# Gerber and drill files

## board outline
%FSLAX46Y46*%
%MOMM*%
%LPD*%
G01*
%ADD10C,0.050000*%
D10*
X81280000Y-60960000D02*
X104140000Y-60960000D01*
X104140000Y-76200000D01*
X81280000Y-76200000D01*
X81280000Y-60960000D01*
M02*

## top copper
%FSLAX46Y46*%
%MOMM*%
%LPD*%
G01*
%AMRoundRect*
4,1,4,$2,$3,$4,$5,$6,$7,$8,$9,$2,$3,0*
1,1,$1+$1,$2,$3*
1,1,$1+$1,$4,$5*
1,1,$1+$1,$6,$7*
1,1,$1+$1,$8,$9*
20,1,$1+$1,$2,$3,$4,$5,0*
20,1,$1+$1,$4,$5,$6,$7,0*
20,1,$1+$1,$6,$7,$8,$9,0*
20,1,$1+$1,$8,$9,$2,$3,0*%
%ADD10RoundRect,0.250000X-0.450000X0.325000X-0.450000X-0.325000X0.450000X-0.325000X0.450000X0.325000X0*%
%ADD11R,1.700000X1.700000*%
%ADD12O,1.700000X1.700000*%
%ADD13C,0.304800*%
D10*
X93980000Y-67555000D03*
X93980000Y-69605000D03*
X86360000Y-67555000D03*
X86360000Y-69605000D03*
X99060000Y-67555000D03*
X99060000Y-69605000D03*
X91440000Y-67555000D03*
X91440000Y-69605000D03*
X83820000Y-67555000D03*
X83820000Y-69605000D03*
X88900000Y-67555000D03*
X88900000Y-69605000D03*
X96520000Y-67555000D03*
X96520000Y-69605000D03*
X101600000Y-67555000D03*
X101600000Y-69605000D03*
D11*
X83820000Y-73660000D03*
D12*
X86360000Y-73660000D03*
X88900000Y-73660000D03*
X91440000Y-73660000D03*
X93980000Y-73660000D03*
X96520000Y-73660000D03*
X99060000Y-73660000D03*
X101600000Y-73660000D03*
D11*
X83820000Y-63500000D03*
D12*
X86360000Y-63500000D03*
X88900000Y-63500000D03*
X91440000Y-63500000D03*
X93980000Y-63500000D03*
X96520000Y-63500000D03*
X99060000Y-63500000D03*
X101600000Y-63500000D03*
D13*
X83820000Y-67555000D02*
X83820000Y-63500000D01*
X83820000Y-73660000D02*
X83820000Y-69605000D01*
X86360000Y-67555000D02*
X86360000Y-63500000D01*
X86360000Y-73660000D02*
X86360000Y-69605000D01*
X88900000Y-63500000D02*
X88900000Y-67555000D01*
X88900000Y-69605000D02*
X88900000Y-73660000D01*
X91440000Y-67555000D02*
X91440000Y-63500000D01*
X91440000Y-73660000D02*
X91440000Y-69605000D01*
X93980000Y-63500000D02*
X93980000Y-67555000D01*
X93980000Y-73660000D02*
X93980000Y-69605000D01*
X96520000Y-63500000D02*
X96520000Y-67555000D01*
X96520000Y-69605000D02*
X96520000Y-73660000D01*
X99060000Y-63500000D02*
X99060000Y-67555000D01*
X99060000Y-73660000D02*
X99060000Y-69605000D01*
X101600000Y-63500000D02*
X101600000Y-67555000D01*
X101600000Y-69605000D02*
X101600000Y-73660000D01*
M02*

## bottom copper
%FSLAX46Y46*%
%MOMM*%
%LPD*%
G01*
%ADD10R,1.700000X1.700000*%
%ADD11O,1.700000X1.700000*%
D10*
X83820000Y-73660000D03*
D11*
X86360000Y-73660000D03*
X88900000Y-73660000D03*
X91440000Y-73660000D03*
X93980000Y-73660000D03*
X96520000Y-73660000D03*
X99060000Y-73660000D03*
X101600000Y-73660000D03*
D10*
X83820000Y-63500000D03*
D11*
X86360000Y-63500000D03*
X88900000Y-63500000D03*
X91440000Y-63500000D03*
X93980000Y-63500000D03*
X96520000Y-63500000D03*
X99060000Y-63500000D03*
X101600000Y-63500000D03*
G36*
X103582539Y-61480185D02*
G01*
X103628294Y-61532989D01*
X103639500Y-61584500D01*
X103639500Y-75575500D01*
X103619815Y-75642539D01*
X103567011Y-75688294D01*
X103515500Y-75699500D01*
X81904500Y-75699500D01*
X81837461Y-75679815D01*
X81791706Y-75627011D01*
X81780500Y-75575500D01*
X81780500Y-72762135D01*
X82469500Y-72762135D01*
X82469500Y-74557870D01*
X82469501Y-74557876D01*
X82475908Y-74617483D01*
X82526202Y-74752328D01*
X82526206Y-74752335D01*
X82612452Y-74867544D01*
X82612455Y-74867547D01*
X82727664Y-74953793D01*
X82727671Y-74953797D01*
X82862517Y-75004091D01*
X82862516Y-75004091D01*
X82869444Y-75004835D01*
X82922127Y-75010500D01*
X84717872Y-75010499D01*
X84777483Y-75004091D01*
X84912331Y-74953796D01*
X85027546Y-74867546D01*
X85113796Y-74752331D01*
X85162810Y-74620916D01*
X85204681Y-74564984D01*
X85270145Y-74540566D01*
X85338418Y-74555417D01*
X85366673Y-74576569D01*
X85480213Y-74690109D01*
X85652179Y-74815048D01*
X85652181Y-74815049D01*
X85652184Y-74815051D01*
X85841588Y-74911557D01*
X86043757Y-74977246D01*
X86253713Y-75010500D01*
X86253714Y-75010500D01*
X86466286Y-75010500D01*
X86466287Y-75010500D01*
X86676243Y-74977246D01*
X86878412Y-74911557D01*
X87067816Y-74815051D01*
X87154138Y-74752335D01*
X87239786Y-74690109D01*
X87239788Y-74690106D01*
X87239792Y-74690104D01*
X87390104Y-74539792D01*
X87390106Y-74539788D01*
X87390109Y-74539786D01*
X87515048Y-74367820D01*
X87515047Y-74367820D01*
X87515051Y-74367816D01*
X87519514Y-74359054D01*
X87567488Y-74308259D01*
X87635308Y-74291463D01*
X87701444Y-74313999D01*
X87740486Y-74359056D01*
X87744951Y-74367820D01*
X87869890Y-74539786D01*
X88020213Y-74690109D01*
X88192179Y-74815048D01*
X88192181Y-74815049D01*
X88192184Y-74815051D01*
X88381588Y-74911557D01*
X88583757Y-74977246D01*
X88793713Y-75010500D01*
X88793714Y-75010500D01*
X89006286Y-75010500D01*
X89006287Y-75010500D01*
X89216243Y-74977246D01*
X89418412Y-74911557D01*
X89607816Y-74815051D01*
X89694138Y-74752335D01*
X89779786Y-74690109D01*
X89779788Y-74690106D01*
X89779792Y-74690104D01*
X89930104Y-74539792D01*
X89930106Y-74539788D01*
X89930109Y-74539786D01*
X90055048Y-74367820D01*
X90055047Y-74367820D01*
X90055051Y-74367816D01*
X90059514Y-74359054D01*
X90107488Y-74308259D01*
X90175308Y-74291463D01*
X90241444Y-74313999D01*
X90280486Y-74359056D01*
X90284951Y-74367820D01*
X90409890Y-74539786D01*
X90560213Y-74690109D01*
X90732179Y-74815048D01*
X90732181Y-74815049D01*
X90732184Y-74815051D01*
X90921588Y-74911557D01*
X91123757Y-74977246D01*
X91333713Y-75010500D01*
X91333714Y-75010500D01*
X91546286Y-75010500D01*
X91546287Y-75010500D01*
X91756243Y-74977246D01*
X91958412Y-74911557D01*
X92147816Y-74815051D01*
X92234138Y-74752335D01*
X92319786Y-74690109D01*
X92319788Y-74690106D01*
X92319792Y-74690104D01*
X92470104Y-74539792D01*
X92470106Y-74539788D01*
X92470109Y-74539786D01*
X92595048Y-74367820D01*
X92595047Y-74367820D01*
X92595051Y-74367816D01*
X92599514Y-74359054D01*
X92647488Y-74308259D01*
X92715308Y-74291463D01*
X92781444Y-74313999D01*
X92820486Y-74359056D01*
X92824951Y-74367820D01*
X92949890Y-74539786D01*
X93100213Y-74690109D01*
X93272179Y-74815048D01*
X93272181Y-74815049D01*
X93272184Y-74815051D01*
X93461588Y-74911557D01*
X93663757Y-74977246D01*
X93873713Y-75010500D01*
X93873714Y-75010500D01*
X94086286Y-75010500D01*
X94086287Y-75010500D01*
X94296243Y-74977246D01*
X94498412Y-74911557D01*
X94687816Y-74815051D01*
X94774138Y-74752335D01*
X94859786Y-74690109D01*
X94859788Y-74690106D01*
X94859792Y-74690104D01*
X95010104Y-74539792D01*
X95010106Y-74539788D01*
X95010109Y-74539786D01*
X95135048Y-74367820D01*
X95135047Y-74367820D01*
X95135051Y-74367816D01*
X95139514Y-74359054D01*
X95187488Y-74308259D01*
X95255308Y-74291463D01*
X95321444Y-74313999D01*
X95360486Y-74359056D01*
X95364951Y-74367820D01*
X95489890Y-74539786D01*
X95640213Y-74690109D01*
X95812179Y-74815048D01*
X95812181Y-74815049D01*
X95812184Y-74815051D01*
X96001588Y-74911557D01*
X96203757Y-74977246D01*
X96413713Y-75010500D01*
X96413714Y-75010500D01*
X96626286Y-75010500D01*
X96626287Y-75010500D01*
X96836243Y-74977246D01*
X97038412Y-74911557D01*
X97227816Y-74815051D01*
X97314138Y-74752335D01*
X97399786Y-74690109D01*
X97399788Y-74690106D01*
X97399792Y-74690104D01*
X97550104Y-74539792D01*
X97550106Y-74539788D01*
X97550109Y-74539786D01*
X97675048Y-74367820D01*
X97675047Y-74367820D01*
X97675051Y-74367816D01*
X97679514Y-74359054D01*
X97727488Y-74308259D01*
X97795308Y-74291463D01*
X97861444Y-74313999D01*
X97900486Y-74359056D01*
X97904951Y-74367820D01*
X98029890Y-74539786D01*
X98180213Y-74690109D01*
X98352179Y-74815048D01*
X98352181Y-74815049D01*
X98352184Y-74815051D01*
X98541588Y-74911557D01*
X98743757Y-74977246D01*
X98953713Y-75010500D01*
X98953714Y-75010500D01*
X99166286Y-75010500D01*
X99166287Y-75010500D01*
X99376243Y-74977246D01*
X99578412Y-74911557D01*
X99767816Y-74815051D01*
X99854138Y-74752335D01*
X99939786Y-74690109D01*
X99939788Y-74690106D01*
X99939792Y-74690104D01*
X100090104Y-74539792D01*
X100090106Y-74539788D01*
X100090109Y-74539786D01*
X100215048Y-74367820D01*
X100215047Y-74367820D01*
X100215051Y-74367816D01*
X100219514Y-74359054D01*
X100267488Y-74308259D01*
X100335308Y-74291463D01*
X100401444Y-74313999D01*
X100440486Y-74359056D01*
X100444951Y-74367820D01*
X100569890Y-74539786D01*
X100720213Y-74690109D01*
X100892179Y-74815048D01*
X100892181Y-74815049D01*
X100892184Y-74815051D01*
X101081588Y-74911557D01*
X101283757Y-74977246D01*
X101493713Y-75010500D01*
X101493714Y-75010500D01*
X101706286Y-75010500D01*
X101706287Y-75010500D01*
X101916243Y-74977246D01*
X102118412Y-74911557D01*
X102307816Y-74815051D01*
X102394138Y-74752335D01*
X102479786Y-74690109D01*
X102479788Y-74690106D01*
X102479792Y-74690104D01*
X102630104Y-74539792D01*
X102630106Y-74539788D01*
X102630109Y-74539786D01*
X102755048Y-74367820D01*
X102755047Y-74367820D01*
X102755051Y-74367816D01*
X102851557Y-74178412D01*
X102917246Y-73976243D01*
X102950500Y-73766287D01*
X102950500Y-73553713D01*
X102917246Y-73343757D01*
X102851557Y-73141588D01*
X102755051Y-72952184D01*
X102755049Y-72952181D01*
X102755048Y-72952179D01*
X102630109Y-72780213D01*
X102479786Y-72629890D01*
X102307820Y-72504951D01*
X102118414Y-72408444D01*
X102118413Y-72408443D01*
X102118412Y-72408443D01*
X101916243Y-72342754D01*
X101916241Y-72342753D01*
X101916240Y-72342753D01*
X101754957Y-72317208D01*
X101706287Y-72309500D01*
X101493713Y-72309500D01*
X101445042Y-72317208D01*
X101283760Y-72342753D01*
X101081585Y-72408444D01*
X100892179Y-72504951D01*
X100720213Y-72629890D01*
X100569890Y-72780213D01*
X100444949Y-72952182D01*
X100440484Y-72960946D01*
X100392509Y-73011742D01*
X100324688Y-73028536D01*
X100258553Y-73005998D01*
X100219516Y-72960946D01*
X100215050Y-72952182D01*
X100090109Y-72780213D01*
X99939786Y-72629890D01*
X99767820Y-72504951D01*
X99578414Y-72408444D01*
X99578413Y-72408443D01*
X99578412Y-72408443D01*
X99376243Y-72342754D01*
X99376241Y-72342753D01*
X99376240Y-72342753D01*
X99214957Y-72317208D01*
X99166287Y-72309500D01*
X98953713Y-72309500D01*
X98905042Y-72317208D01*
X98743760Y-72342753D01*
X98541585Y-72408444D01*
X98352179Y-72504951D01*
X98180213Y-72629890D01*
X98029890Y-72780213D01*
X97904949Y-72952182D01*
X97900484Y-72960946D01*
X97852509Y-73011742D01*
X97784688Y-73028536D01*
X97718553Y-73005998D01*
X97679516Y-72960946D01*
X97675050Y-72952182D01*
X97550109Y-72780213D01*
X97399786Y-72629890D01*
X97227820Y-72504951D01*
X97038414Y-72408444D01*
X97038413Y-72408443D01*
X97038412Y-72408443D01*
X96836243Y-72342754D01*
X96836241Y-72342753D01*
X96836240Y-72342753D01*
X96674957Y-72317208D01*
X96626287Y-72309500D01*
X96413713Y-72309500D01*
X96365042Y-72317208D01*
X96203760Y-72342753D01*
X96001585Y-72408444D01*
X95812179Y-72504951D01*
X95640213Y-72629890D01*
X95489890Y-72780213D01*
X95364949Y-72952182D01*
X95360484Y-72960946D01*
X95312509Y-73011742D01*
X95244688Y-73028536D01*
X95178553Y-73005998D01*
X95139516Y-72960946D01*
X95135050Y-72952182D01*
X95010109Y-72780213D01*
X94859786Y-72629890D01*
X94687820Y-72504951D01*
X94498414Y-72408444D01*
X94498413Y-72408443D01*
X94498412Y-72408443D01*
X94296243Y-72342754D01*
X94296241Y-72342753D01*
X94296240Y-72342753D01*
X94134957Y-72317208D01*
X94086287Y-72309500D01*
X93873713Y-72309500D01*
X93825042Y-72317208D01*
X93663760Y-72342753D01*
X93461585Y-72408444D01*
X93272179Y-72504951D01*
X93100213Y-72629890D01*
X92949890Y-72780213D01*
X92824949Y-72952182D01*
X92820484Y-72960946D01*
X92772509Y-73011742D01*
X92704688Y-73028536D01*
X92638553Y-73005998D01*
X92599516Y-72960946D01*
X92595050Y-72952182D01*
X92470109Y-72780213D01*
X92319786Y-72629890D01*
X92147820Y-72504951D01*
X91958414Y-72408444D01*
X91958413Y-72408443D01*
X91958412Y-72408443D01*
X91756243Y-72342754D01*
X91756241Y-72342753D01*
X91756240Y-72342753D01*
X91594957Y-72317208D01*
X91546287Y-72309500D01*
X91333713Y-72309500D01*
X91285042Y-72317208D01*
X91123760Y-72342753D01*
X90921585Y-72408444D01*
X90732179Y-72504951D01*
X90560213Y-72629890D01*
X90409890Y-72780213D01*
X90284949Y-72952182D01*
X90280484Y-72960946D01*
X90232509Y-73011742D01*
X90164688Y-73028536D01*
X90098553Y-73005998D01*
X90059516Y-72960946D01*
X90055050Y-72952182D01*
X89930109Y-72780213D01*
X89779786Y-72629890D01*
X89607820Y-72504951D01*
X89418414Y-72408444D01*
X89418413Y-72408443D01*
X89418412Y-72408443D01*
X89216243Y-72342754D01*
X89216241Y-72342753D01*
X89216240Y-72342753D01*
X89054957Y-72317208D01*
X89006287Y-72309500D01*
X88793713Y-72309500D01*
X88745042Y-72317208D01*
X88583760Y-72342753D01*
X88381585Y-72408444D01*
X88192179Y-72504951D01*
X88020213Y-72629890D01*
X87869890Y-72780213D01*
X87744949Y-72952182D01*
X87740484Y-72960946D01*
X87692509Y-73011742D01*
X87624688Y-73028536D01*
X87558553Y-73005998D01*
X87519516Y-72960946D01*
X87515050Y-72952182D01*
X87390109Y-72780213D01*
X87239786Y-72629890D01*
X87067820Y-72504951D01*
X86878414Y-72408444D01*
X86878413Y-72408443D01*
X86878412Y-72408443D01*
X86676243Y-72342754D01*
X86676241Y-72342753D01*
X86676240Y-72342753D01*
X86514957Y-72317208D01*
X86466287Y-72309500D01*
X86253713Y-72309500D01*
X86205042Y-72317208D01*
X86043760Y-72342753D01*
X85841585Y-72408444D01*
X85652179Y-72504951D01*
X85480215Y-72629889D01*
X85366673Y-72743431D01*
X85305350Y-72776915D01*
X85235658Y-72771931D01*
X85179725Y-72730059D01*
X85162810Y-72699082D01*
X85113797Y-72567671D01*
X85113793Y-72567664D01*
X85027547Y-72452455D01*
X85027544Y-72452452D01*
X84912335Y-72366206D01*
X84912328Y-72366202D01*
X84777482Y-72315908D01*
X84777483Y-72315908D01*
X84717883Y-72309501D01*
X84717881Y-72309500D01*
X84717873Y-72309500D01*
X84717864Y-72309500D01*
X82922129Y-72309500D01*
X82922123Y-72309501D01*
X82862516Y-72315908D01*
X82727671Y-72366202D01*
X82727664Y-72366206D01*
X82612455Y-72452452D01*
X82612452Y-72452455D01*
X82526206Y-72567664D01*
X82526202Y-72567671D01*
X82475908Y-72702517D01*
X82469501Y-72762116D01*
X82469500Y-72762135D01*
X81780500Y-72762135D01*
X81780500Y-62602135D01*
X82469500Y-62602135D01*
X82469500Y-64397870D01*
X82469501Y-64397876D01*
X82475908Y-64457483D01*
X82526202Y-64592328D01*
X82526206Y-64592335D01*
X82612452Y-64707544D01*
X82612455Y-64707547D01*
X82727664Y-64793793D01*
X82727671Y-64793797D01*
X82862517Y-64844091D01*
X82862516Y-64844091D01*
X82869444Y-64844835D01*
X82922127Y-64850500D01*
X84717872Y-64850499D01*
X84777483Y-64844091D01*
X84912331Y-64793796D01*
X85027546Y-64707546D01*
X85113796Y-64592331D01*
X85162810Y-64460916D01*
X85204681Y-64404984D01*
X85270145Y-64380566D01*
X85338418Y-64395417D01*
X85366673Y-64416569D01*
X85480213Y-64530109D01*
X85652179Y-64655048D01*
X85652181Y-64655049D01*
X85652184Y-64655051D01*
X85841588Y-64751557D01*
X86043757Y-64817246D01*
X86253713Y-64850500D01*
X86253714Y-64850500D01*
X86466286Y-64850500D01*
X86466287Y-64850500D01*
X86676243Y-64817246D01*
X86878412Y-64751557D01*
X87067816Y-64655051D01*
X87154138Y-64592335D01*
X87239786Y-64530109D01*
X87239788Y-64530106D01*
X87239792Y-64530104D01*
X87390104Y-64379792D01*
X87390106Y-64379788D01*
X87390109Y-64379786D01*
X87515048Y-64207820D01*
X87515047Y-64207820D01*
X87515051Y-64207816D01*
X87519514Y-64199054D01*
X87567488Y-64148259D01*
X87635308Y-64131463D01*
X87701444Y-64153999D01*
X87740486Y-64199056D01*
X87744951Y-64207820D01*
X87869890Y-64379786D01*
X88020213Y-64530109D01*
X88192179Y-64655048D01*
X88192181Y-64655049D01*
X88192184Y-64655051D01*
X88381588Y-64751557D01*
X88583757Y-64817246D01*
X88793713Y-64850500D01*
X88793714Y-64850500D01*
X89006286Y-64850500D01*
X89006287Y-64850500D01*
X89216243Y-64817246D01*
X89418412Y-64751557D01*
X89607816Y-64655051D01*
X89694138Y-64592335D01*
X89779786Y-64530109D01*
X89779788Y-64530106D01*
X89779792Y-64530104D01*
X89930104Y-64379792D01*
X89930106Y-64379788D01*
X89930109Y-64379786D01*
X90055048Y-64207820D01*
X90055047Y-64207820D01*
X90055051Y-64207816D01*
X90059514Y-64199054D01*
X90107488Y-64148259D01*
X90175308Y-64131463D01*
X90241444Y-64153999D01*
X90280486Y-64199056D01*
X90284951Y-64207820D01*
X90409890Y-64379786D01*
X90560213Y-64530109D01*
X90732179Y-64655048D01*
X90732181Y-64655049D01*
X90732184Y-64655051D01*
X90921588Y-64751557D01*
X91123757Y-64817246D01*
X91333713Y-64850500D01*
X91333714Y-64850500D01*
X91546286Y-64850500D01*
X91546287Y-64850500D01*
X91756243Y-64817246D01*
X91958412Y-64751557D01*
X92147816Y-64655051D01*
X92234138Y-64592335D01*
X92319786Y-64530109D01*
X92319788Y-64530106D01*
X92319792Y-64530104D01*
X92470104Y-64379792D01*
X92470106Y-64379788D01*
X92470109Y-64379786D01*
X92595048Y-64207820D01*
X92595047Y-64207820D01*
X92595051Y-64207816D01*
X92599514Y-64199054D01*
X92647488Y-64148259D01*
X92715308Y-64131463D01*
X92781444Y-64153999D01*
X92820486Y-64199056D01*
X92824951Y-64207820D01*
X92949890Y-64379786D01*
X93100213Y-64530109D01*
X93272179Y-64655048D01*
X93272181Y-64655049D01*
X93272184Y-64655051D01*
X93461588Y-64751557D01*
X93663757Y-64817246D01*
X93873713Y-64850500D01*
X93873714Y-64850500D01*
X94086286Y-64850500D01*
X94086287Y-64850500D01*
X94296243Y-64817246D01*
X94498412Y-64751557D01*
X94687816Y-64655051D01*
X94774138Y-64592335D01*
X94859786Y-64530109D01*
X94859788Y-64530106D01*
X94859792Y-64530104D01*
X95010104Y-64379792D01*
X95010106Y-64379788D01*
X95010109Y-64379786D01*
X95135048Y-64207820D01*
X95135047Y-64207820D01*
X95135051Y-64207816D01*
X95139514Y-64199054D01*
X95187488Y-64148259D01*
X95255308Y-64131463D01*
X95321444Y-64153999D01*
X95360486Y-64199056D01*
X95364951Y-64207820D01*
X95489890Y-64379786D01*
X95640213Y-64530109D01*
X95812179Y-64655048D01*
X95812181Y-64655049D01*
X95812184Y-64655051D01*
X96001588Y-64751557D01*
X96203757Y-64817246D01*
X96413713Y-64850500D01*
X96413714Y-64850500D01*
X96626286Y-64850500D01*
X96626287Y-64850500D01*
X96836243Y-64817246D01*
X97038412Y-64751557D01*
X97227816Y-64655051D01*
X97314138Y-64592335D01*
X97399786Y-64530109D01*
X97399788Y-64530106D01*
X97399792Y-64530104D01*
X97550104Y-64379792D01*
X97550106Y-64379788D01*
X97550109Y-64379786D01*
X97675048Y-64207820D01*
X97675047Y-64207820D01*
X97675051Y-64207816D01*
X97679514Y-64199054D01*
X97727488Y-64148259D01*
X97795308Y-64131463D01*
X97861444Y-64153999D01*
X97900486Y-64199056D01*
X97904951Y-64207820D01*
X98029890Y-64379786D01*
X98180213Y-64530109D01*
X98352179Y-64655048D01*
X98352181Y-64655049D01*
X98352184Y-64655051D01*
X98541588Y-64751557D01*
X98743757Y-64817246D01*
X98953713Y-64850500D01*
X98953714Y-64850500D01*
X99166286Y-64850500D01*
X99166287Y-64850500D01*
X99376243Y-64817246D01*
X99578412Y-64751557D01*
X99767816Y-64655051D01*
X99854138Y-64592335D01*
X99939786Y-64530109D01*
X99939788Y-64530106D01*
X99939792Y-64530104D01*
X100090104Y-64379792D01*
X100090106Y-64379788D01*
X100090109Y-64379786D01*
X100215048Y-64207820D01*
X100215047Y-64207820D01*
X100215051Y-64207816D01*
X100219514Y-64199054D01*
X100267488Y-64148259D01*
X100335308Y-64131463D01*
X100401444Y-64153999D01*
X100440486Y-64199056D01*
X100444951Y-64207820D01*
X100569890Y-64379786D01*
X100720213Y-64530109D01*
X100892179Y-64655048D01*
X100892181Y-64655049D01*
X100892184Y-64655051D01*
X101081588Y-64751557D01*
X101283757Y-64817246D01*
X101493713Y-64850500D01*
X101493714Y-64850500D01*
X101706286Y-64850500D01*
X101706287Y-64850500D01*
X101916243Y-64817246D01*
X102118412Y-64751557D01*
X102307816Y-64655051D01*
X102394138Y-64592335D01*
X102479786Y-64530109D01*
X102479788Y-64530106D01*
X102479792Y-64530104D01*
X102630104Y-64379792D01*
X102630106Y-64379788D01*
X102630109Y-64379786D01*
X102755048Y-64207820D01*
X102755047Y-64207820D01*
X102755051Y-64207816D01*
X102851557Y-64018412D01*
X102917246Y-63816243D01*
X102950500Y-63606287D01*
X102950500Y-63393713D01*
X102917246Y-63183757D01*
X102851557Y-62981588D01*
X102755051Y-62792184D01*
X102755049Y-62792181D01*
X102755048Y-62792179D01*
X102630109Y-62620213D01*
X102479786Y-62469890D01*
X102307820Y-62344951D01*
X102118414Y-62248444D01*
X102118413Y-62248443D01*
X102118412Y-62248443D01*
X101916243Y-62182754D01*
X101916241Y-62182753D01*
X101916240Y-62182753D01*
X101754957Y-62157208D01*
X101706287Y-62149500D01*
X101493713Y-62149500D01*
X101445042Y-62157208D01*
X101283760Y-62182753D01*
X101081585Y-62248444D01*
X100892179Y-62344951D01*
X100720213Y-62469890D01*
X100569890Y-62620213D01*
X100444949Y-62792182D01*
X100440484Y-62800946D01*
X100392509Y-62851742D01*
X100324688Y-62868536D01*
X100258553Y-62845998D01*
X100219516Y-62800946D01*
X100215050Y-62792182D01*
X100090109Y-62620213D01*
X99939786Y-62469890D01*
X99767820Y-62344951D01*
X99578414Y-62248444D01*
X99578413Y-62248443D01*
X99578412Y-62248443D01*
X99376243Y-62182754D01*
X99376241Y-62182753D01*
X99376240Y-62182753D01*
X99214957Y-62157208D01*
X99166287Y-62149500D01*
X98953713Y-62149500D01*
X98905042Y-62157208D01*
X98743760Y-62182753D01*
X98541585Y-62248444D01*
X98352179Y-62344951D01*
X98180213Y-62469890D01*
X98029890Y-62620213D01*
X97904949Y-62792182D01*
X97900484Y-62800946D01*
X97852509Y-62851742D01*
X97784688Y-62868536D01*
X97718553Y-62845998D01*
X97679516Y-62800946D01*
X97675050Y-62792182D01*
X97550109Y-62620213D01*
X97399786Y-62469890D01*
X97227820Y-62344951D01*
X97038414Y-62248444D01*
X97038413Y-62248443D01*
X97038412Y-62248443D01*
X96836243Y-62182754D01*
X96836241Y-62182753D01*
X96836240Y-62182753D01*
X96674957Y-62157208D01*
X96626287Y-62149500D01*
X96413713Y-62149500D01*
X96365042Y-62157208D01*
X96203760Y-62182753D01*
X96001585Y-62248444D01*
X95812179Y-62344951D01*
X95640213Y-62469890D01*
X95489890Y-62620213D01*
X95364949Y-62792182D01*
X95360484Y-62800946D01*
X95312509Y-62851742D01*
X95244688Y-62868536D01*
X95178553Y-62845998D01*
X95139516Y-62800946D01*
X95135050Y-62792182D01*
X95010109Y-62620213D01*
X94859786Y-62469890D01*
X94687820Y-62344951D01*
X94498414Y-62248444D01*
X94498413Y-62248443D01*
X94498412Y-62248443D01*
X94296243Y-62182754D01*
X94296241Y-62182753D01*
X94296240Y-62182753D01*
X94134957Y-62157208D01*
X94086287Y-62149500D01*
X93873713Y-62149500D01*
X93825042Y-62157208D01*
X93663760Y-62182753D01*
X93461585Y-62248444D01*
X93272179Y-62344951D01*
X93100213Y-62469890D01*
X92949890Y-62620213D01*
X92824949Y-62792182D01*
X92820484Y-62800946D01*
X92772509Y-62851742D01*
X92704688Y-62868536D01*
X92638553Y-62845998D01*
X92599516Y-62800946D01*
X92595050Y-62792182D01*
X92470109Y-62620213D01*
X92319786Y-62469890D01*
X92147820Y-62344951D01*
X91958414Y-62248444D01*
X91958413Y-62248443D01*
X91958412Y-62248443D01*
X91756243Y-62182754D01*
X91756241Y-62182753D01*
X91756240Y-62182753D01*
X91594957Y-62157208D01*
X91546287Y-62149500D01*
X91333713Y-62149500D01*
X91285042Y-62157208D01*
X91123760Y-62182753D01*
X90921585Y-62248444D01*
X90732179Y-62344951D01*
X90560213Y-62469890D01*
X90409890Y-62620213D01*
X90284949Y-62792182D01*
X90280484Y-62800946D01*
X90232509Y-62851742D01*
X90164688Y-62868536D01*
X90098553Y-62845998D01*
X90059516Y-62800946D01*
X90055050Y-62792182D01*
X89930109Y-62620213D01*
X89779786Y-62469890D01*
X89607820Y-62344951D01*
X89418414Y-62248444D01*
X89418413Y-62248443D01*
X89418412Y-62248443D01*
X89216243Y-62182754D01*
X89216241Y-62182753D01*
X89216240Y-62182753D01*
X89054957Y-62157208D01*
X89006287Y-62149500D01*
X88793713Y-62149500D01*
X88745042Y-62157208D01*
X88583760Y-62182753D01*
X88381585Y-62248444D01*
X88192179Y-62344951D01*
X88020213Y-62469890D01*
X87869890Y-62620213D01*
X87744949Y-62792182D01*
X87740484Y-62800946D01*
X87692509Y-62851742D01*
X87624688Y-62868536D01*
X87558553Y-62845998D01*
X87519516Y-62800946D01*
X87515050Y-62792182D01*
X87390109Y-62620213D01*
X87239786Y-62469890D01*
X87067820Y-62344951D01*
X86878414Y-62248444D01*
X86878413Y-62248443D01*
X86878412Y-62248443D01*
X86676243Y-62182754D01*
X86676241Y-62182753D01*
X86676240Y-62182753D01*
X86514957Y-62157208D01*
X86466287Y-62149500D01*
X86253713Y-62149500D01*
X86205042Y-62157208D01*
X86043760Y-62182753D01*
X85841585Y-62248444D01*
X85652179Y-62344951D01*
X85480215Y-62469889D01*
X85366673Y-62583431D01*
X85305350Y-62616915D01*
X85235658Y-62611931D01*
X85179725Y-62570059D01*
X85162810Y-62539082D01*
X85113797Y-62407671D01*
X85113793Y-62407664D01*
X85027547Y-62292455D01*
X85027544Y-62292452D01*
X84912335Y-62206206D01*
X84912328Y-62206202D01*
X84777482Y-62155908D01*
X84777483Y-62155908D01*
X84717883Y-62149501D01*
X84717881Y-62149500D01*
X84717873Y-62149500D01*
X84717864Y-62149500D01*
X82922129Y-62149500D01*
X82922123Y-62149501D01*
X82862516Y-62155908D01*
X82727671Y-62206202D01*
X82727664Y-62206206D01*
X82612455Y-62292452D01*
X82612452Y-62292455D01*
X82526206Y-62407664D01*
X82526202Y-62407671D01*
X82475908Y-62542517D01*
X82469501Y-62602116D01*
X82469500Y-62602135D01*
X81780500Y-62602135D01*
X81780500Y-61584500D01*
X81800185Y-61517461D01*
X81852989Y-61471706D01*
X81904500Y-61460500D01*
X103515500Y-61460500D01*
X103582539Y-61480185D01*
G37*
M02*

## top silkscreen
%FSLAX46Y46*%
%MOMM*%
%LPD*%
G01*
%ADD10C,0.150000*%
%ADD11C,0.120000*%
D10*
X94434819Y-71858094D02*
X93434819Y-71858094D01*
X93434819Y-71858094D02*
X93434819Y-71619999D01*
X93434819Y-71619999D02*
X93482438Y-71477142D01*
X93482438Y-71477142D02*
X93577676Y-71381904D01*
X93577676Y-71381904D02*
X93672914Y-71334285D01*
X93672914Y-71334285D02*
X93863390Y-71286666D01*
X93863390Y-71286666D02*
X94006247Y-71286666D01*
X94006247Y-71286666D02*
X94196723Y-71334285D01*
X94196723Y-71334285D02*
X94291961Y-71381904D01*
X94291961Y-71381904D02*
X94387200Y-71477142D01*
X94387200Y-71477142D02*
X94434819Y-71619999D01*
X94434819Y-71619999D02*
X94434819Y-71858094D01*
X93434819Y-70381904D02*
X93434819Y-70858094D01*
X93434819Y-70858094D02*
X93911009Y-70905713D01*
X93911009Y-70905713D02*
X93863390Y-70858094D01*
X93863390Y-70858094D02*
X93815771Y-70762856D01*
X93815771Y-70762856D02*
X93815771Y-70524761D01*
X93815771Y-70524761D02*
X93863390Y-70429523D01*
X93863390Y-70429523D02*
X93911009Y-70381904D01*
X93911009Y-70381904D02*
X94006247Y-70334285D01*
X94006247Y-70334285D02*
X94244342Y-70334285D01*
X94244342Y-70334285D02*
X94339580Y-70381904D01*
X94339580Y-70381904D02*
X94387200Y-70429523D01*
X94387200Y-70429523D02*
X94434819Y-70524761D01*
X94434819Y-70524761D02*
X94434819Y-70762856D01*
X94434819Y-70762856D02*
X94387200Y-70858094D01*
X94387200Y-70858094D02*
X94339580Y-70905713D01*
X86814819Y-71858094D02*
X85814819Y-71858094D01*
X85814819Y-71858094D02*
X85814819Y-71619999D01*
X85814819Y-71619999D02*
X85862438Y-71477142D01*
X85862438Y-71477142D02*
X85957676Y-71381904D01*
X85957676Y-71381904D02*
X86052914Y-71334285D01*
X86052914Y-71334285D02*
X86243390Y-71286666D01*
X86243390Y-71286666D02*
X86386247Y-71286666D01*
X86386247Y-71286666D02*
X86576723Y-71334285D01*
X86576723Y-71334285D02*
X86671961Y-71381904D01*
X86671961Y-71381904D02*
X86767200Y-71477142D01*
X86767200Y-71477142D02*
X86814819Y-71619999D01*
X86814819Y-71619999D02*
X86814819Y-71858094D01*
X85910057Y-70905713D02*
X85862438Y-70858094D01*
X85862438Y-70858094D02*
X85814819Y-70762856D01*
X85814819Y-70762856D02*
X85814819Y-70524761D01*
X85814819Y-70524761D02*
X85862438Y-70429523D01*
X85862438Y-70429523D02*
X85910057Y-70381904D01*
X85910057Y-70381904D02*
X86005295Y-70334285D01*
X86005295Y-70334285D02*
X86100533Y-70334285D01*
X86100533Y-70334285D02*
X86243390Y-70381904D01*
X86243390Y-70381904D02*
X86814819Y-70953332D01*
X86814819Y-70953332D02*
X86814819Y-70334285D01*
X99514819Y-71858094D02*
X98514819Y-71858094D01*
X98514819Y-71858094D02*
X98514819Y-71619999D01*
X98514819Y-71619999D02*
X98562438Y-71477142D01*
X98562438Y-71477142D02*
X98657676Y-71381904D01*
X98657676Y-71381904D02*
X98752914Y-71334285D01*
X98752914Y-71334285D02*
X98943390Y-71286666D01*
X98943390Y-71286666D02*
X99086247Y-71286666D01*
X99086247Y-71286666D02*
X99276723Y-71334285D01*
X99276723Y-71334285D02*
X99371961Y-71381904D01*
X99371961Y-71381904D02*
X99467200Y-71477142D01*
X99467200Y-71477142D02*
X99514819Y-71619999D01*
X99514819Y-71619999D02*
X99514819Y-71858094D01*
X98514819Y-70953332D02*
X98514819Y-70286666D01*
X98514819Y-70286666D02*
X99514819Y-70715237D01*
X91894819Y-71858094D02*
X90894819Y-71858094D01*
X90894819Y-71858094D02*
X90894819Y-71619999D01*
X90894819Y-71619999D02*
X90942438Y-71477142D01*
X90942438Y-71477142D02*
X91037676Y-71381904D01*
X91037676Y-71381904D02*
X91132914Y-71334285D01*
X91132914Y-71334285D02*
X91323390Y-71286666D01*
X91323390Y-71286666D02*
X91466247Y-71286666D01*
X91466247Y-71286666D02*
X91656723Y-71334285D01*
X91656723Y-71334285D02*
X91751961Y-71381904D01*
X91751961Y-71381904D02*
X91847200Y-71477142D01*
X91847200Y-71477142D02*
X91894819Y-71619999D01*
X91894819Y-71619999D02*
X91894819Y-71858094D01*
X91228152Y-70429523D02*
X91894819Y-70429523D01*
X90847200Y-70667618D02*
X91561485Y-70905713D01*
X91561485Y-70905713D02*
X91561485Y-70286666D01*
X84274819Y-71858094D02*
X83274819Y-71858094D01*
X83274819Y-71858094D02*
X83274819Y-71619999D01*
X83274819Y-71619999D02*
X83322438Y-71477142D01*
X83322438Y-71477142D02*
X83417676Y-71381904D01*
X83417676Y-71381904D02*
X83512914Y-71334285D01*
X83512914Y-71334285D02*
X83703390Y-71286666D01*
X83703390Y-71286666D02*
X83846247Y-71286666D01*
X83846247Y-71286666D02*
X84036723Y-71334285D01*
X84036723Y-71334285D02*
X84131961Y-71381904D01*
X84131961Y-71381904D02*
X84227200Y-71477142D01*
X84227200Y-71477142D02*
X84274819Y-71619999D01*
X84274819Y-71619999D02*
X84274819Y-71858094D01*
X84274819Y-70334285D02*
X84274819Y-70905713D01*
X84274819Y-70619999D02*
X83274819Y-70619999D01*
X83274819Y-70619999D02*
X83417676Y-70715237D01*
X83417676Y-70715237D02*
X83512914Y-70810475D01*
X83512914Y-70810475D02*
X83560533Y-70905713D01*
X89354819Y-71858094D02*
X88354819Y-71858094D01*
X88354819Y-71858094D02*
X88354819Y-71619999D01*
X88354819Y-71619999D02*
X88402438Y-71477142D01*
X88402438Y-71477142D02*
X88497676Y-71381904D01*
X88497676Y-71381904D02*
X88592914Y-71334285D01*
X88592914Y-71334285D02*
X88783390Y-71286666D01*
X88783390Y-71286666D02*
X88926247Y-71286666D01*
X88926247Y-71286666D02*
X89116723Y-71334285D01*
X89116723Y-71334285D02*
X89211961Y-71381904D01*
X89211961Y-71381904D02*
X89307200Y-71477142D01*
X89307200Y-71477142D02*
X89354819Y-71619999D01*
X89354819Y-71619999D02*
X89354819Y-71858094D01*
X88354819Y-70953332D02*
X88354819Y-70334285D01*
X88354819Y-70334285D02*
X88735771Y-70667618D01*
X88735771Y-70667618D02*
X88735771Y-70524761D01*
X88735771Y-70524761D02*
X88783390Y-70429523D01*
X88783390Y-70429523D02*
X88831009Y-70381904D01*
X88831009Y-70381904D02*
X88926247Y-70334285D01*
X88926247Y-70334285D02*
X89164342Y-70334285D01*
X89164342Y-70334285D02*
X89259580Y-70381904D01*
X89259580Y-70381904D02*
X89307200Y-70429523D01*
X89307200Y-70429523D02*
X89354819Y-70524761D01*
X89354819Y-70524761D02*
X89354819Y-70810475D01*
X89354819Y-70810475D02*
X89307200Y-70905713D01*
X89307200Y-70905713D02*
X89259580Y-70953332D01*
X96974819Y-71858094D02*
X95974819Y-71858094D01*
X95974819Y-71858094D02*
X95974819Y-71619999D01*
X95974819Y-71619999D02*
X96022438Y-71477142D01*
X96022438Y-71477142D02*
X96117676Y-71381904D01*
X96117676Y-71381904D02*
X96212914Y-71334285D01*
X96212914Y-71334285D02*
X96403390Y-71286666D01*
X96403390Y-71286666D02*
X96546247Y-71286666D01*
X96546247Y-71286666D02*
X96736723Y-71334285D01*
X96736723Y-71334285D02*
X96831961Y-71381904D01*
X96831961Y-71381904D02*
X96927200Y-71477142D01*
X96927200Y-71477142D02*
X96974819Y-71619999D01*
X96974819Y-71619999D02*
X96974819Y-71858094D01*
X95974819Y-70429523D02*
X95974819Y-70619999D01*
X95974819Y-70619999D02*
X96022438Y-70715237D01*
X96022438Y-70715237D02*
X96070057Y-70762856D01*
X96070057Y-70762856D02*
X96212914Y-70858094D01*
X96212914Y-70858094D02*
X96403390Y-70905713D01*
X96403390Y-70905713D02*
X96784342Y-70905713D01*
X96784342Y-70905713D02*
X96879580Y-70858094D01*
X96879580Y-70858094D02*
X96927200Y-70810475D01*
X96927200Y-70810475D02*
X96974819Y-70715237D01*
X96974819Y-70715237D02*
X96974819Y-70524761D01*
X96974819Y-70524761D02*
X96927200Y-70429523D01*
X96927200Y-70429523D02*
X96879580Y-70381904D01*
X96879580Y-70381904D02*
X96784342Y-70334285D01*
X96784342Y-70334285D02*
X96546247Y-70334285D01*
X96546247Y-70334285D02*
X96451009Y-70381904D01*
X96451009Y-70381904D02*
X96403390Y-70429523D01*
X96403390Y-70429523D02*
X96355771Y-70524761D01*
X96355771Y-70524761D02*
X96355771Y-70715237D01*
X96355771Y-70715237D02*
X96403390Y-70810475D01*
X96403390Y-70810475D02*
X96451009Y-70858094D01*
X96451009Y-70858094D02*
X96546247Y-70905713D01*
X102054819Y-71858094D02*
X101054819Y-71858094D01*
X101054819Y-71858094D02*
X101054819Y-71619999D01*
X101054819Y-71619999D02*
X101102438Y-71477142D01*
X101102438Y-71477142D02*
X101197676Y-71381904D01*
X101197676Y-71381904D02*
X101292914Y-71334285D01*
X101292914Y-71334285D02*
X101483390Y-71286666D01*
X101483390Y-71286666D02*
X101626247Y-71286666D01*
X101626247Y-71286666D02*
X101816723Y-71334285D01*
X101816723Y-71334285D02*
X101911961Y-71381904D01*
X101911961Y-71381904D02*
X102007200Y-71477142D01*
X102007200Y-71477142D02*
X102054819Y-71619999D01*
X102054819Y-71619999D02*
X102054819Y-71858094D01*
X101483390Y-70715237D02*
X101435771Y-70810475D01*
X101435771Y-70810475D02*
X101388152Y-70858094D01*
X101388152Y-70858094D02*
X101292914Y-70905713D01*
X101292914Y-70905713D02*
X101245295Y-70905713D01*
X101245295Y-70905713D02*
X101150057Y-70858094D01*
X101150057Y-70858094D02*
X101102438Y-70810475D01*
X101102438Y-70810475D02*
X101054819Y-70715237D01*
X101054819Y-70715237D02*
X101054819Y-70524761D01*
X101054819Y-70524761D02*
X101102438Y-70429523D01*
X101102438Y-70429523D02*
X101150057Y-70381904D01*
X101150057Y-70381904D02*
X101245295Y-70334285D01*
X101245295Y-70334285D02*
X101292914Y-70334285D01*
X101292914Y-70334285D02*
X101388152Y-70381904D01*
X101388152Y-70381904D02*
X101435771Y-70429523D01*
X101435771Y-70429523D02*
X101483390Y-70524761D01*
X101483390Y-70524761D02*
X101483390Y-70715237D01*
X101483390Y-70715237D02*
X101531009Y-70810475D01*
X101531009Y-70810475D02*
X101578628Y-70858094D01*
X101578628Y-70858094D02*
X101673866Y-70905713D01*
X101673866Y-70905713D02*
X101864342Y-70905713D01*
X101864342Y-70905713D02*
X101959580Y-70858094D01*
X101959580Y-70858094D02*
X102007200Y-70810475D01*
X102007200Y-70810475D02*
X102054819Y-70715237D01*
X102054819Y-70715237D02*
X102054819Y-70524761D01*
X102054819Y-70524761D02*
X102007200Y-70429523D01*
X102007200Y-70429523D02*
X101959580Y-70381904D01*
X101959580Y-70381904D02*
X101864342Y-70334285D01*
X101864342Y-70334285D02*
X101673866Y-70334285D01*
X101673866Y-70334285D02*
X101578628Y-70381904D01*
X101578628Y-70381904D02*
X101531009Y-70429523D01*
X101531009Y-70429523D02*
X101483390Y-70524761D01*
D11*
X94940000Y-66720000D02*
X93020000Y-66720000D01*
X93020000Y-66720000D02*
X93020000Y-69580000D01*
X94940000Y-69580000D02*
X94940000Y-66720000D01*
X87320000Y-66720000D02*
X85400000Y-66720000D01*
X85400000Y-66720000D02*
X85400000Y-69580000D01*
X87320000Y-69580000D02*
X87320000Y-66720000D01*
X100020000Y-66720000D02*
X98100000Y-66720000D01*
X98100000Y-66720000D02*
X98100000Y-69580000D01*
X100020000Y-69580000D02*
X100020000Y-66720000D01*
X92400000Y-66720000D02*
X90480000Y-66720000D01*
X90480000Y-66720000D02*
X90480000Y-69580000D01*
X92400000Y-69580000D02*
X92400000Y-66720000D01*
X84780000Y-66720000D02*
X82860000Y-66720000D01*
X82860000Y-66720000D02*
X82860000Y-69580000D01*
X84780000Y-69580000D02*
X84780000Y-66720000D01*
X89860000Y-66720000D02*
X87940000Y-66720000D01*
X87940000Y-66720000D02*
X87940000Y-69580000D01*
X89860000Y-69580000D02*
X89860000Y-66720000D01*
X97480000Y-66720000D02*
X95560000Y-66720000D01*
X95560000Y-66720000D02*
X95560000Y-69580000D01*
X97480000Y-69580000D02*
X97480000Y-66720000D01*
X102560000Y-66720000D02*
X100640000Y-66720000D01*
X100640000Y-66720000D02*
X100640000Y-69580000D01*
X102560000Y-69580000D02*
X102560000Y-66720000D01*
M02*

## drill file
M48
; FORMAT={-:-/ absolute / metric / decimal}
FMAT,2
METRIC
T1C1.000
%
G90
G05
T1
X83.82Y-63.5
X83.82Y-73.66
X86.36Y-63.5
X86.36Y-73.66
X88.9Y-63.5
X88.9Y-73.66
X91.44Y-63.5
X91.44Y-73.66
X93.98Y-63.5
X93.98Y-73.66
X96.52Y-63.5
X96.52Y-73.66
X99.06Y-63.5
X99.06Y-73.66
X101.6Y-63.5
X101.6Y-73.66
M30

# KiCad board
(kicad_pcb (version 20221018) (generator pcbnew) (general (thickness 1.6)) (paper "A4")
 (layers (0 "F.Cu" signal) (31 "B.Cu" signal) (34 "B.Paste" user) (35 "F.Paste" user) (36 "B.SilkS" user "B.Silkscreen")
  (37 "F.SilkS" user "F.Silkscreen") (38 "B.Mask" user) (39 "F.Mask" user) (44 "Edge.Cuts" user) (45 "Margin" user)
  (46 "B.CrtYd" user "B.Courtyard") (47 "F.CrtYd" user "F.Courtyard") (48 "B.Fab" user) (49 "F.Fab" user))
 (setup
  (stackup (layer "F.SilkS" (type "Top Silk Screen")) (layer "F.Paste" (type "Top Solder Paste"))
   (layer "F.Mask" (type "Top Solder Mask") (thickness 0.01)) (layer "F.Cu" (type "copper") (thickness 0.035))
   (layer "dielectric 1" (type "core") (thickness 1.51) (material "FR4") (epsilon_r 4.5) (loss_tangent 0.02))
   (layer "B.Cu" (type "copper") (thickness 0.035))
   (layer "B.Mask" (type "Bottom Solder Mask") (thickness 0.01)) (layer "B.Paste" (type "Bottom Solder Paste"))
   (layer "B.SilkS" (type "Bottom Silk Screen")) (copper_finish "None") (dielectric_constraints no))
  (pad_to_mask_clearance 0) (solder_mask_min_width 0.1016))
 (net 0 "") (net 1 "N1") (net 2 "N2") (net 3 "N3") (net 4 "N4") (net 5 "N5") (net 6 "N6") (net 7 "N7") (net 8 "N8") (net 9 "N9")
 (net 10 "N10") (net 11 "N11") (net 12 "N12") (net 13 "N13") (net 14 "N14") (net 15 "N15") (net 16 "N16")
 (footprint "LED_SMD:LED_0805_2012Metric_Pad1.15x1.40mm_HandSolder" (layer "F.Cu") (at 93.98 68.58 -90)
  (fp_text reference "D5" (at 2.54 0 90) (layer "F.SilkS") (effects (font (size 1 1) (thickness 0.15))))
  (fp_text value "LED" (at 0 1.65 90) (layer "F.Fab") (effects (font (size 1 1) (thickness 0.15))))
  (fp_line (start -1.86 -0.96) (end -1.86 0.96) (stroke (width 0.12) (type solid)) (layer "F.SilkS"))
  (fp_line (start -1.86 0.96) (end 1 0.96) (stroke (width 0.12) (type solid)) (layer "F.SilkS"))
  (fp_line (start 1 -0.96) (end -1.86 -0.96) (stroke (width 0.12) (type solid)) (layer "F.SilkS"))
  (pad "1" smd roundrect (at -1.025 0 270) (size 1.15 1.4) (layers "F.Cu" "F.Paste" "F.Mask") (roundrect_rratio 0.217391) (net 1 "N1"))
  (pad "2" smd roundrect (at 1.025 0 270) (size 1.15 1.4) (layers "F.Cu" "F.Paste" "F.Mask") (roundrect_rratio 0.217391) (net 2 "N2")))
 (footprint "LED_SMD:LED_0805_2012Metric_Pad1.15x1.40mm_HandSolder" (layer "F.Cu") (at 86.36 68.58 -90)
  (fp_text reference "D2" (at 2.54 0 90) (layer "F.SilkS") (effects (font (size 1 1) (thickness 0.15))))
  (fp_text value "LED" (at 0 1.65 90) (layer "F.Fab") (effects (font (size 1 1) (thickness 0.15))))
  (fp_line (start -1.86 -0.96) (end -1.86 0.96) (stroke (width 0.12) (type solid)) (layer "F.SilkS"))
  (fp_line (start -1.86 0.96) (end 1 0.96) (stroke (width 0.12) (type solid)) (layer "F.SilkS"))
  (fp_line (start 1 -0.96) (end -1.86 -0.96) (stroke (width 0.12) (type solid)) (layer "F.SilkS"))
  (pad "1" smd roundrect (at -1.025 0 270) (size 1.15 1.4) (layers "F.Cu" "F.Paste" "F.Mask") (roundrect_rratio 0.217391) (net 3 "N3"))
  (pad "2" smd roundrect (at 1.025 0 270) (size 1.15 1.4) (layers "F.Cu" "F.Paste" "F.Mask") (roundrect_rratio 0.217391) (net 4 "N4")))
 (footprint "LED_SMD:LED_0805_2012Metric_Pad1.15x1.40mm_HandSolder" (layer "F.Cu") (at 99.06 68.58 -90)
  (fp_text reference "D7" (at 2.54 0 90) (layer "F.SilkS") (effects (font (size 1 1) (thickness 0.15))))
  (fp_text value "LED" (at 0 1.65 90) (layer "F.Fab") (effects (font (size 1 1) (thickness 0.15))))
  (fp_line (start -1.86 -0.96) (end -1.86 0.96) (stroke (width 0.12) (type solid)) (layer "F.SilkS"))
  (fp_line (start -1.86 0.96) (end 1 0.96) (stroke (width 0.12) (type solid)) (layer "F.SilkS"))
  (fp_line (start 1 -0.96) (end -1.86 -0.96) (stroke (width 0.12) (type solid)) (layer "F.SilkS"))
  (pad "1" smd roundrect (at -1.025 0 270) (size 1.15 1.4) (layers "F.Cu" "F.Paste" "F.Mask") (roundrect_rratio 0.217391) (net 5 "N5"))
  (pad "2" smd roundrect (at 1.025 0 270) (size 1.15 1.4) (layers "F.Cu" "F.Paste" "F.Mask") (roundrect_rratio 0.217391) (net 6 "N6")))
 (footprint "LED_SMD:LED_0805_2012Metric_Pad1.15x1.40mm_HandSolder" (layer "F.Cu") (at 91.44 68.58 -90)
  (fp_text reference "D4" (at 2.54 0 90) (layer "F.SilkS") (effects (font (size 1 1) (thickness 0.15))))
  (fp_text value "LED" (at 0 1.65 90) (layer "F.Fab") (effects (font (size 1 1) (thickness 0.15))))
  (fp_line (start -1.86 -0.96) (end -1.86 0.96) (stroke (width 0.12) (type solid)) (layer "F.SilkS"))
  (fp_line (start -1.86 0.96) (end 1 0.96) (stroke (width 0.12) (type solid)) (layer "F.SilkS"))
  (fp_line (start 1 -0.96) (end -1.86 -0.96) (stroke (width 0.12) (type solid)) (layer "F.SilkS"))
  (pad "1" smd roundrect (at -1.025 0 270) (size 1.15 1.4) (layers "F.Cu" "F.Paste" "F.Mask") (roundrect_rratio 0.217391) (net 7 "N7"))
  (pad "2" smd roundrect (at 1.025 0 270) (size 1.15 1.4) (layers "F.Cu" "F.Paste" "F.Mask") (roundrect_rratio 0.217391) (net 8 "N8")))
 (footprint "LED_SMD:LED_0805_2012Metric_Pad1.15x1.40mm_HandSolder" (layer "F.Cu") (at 83.82 68.58 -90)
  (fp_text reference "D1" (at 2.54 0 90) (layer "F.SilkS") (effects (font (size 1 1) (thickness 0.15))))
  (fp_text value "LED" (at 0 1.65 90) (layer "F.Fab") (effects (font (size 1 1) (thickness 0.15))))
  (fp_line (start -1.86 -0.96) (end -1.86 0.96) (stroke (width 0.12) (type solid)) (layer "F.SilkS"))
  (fp_line (start -1.86 0.96) (end 1 0.96) (stroke (width 0.12) (type solid)) (layer "F.SilkS"))
  (fp_line (start 1 -0.96) (end -1.86 -0.96) (stroke (width 0.12) (type solid)) (layer "F.SilkS"))
  (pad "1" smd roundrect (at -1.025 0 270) (size 1.15 1.4) (layers "F.Cu" "F.Paste" "F.Mask") (roundrect_rratio 0.217391) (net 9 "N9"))
  (pad "2" smd roundrect (at 1.025 0 270) (size 1.15 1.4) (layers "F.Cu" "F.Paste" "F.Mask") (roundrect_rratio 0.217391) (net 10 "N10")))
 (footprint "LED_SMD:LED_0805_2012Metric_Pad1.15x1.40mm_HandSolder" (layer "F.Cu") (at 88.9 68.58 -90)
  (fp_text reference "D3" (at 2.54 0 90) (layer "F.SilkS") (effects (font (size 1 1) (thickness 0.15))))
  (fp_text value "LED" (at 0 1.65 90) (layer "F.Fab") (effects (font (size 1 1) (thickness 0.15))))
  (fp_line (start -1.86 -0.96) (end -1.86 0.96) (stroke (width 0.12) (type solid)) (layer "F.SilkS"))
  (fp_line (start -1.86 0.96) (end 1 0.96) (stroke (width 0.12) (type solid)) (layer "F.SilkS"))
  (fp_line (start 1 -0.96) (end -1.86 -0.96) (stroke (width 0.12) (type solid)) (layer "F.SilkS"))
  (pad "1" smd roundrect (at -1.025 0 270) (size 1.15 1.4) (layers "F.Cu" "F.Paste" "F.Mask") (roundrect_rratio 0.217391) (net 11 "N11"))
  (pad "2" smd roundrect (at 1.025 0 270) (size 1.15 1.4) (layers "F.Cu" "F.Paste" "F.Mask") (roundrect_rratio 0.217391) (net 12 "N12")))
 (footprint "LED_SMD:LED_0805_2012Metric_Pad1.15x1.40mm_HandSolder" (layer "F.Cu") (at 96.52 68.58 -90)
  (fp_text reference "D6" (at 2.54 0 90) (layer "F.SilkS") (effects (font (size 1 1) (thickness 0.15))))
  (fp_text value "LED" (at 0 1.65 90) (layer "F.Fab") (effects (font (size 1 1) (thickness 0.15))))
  (fp_line (start -1.86 -0.96) (end -1.86 0.96) (stroke (width 0.12) (type solid)) (layer "F.SilkS"))
  (fp_line (start -1.86 0.96) (end 1 0.96) (stroke (width 0.12) (type solid)) (layer "F.SilkS"))
  (fp_line (start 1 -0.96) (end -1.86 -0.96) (stroke (width 0.12) (type solid)) (layer "F.SilkS"))
  (pad "1" smd roundrect (at -1.025 0 270) (size 1.15 1.4) (layers "F.Cu" "F.Paste" "F.Mask") (roundrect_rratio 0.217391) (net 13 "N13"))
  (pad "2" smd roundrect (at 1.025 0 270) (size 1.15 1.4) (layers "F.Cu" "F.Paste" "F.Mask") (roundrect_rratio 0.217391) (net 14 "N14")))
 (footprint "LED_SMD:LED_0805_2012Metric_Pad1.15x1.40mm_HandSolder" (layer "F.Cu") (at 101.6 68.58 -90)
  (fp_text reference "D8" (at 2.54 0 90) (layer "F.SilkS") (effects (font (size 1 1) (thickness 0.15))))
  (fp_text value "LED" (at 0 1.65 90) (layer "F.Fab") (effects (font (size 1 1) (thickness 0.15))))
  (fp_line (start -1.86 -0.96) (end -1.86 0.96) (stroke (width 0.12) (type solid)) (layer "F.SilkS"))
  (fp_line (start -1.86 0.96) (end 1 0.96) (stroke (width 0.12) (type solid)) (layer "F.SilkS"))
  (fp_line (start 1 -0.96) (end -1.86 -0.96) (stroke (width 0.12) (type solid)) (layer "F.SilkS"))
  (pad "1" smd roundrect (at -1.025 0 270) (size 1.15 1.4) (layers "F.Cu" "F.Paste" "F.Mask") (roundrect_rratio 0.217391) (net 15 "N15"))
  (pad "2" smd roundrect (at 1.025 0 270) (size 1.15 1.4) (layers "F.Cu" "F.Paste" "F.Mask") (roundrect_rratio 0.217391) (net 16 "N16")))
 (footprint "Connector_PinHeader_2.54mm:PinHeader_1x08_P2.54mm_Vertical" (layer "B.Cu") (at 83.82 73.66 -90)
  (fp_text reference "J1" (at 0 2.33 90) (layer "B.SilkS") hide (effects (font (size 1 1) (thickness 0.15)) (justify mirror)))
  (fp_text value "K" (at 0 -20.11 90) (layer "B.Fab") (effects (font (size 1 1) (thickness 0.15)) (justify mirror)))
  (pad "1" thru_hole rect (at 0 0 270) (size 1.7 1.7) (drill 1) (layers "*.Cu" "*.Mask") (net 10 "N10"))
  (pad "2" thru_hole oval (at 0 -2.54 270) (size 1.7 1.7) (drill 1) (layers "*.Cu" "*.Mask") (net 4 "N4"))
  (pad "3" thru_hole oval (at 0 -5.08 270) (size 1.7 1.7) (drill 1) (layers "*.Cu" "*.Mask") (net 12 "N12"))
  (pad "4" thru_hole oval (at 0 -7.62 270) (size 1.7 1.7) (drill 1) (layers "*.Cu" "*.Mask") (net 8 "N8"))
  (pad "5" thru_hole oval (at 0 -10.16 270) (size 1.7 1.7) (drill 1) (layers "*.Cu" "*.Mask") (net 2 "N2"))
  (pad "6" thru_hole oval (at 0 -12.7 270) (size 1.7 1.7) (drill 1) (layers "*.Cu" "*.Mask") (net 14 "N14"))
  (pad "7" thru_hole oval (at 0 -15.24 270) (size 1.7 1.7) (drill 1) (layers "*.Cu" "*.Mask") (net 6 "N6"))
  (pad "8" thru_hole oval (at 0 -17.78 270) (size 1.7 1.7) (drill 1) (layers "*.Cu" "*.Mask") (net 16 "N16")))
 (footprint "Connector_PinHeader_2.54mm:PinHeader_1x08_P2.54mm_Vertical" (layer "B.Cu") (at 83.82 63.5 -90)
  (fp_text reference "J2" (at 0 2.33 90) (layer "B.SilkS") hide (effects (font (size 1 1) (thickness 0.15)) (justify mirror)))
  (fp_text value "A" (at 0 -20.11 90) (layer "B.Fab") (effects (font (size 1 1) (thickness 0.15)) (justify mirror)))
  (pad "1" thru_hole rect (at 0 0 270) (size 1.7 1.7) (drill 1) (layers "*.Cu" "*.Mask") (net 9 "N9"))
  (pad "2" thru_hole oval (at 0 -2.54 270) (size 1.7 1.7) (drill 1) (layers "*.Cu" "*.Mask") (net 3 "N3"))
  (pad "3" thru_hole oval (at 0 -5.08 270) (size 1.7 1.7) (drill 1) (layers "*.Cu" "*.Mask") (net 11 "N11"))
  (pad "4" thru_hole oval (at 0 -7.62 270) (size 1.7 1.7) (drill 1) (layers "*.Cu" "*.Mask") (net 7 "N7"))
  (pad "5" thru_hole oval (at 0 -10.16 270) (size 1.7 1.7) (drill 1) (layers "*.Cu" "*.Mask") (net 1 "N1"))
  (pad "6" thru_hole oval (at 0 -12.7 270) (size 1.7 1.7) (drill 1) (layers "*.Cu" "*.Mask") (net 13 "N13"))
  (pad "7" thru_hole oval (at 0 -15.24 270) (size 1.7 1.7) (drill 1) (layers "*.Cu" "*.Mask") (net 5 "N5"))
  (pad "8" thru_hole oval (at 0 -17.78 270) (size 1.7 1.7) (drill 1) (layers "*.Cu" "*.Mask") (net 15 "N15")))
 (gr_rect (start 81.28 60.96) (end 104.14 76.2) (stroke (width 0.05) (type default)) (fill none) (layer "Edge.Cuts"))
 (segment (start 83.82 67.555) (end 83.82 63.5) (width 0.3048) (layer "F.Cu") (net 9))
 (segment (start 83.82 73.66) (end 83.82 69.605) (width 0.3048) (layer "F.Cu") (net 10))
 (segment (start 86.36 67.555) (end 86.36 63.5) (width 0.3048) (layer "F.Cu") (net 3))
 (segment (start 86.36 73.66) (end 86.36 69.605) (width 0.3048) (layer "F.Cu") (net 4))
 (segment (start 88.9 63.5) (end 88.9 67.555) (width 0.3048) (layer "F.Cu") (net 11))
 (segment (start 88.9 69.605) (end 88.9 73.66) (width 0.3048) (layer "F.Cu") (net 12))
 (segment (start 91.44 67.555) (end 91.44 63.5) (width 0.3048) (layer "F.Cu") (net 7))
 (segment (start 91.44 73.66) (end 91.44 69.605) (width 0.3048) (layer "F.Cu") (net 8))
 (segment (start 93.98 63.5) (end 93.98 67.555) (width 0.3048) (layer "F.Cu") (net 1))
 (segment (start 93.98 73.66) (end 93.98 69.605) (width 0.3048) (layer "F.Cu") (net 2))
 (segment (start 96.52 63.5) (end 96.52 67.555) (width 0.3048) (layer "F.Cu") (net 13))
 (segment (start 96.52 69.605) (end 96.52 73.66) (width 0.3048) (layer "F.Cu") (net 14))
 (segment (start 99.06 63.5) (end 99.06 67.555) (width 0.3048) (layer "F.Cu") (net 5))
 (segment (start 99.06 73.66) (end 99.06 69.605) (width 0.3048) (layer "F.Cu") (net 6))
 (segment (start 101.6 63.5) (end 101.6 67.555) (width 0.3048) (layer "F.Cu") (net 15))
 (segment (start 101.6 69.605) (end 101.6 73.66) (width 0.3048) (layer "F.Cu") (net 16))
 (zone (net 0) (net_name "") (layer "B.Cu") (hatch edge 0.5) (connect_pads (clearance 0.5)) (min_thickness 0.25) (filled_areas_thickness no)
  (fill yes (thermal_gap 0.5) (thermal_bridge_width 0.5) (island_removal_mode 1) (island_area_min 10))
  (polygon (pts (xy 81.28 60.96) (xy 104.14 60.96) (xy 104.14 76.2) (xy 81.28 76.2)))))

